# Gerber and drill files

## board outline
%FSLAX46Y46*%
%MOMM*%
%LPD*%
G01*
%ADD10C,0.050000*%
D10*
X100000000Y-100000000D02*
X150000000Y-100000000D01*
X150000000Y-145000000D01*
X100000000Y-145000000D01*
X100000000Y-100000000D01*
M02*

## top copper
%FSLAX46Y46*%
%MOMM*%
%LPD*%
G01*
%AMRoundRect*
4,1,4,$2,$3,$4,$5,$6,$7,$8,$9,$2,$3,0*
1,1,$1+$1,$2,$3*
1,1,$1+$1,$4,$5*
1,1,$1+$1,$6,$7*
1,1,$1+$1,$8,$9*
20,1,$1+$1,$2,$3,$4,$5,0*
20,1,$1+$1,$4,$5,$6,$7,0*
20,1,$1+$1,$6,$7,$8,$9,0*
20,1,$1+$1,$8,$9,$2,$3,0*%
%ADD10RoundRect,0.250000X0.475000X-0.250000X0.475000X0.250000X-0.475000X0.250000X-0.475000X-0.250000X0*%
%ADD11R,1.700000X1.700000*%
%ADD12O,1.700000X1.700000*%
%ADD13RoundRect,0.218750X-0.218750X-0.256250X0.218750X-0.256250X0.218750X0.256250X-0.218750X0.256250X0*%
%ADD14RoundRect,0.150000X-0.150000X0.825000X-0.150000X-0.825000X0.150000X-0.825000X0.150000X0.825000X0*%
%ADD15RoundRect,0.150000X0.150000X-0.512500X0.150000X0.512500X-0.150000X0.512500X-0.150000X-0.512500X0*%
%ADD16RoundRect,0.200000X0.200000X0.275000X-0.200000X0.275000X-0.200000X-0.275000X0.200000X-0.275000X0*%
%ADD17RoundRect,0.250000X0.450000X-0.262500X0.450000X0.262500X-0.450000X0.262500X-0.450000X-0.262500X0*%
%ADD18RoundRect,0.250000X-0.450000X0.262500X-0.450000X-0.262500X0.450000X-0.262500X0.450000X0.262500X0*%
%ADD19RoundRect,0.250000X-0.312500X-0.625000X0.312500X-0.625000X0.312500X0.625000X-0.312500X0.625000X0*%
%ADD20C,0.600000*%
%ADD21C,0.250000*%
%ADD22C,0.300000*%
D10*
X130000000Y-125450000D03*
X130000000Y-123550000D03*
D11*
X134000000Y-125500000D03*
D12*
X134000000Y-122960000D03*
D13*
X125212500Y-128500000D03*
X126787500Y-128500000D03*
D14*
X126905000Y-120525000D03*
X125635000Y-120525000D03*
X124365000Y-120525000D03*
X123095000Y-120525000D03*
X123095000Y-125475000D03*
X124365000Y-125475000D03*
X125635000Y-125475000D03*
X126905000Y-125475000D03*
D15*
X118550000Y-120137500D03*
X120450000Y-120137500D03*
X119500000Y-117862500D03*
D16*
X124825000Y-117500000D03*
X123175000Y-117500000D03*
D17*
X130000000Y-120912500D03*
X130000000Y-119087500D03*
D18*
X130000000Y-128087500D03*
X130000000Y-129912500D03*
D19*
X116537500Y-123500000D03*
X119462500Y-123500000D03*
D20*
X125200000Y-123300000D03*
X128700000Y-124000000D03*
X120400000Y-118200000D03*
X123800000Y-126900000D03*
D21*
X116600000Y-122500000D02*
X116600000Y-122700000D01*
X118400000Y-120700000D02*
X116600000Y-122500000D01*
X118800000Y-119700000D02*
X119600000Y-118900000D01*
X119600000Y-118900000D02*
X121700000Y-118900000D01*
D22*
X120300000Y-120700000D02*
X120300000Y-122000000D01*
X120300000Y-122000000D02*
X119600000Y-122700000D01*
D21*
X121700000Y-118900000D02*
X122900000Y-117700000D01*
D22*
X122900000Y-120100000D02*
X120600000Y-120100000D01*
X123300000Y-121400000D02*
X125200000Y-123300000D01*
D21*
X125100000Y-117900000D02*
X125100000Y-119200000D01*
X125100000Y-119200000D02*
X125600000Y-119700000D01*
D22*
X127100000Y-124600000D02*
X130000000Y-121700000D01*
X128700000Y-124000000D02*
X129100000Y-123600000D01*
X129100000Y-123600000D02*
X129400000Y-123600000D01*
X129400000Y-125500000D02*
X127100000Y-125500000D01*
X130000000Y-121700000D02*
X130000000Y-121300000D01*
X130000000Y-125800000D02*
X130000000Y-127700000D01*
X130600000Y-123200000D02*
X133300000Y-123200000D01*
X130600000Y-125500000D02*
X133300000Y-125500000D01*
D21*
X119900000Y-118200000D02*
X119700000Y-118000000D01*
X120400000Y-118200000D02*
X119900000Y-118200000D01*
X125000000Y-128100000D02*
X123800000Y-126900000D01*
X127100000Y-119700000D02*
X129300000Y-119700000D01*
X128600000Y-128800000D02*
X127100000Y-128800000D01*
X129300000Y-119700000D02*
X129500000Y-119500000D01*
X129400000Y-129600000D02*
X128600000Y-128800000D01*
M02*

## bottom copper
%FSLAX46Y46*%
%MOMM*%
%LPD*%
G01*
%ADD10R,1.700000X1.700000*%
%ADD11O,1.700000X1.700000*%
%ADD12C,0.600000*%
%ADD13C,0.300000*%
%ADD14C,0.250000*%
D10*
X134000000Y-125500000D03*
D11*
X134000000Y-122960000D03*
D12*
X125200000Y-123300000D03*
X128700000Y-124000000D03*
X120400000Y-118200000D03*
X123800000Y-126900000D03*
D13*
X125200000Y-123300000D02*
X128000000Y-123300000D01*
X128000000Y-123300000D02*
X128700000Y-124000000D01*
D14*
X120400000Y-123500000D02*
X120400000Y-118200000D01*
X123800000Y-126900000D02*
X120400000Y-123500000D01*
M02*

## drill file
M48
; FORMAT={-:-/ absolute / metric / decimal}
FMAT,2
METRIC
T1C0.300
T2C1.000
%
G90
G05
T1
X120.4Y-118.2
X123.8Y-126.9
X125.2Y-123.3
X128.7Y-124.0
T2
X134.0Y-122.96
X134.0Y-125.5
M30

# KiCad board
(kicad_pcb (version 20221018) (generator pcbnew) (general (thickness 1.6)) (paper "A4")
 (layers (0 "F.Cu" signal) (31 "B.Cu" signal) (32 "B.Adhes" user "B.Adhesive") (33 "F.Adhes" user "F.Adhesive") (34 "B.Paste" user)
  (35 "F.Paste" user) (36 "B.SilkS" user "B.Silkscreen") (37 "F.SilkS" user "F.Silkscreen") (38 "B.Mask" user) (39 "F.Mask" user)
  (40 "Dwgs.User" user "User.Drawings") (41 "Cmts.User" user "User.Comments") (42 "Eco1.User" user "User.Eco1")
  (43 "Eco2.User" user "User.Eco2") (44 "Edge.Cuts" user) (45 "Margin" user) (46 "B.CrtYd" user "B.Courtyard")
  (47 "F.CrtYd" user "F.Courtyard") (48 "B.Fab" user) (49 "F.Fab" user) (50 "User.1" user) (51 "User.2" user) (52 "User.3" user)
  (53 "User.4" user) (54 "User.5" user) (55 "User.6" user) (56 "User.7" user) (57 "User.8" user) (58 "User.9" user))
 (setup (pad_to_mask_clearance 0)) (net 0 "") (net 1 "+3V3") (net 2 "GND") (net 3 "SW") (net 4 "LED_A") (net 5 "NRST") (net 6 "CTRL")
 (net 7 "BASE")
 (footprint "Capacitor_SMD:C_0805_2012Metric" (layer "F.Cu") (at 130 124.5 90)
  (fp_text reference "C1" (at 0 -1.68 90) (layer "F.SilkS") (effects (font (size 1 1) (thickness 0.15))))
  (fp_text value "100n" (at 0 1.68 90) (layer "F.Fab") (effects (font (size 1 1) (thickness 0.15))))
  (pad "1" smd roundrect (at -0.95 0 90) (size 1 1.45) (layers "F.Cu" "F.Paste" "F.Mask") (roundrect_rratio 0.25) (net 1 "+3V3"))
  (pad "2" smd roundrect (at 0.95 0 90) (size 1 1.45) (layers "F.Cu" "F.Paste" "F.Mask") (roundrect_rratio 0.25) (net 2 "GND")))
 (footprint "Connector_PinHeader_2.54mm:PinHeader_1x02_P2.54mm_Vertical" (layer "F.Cu") (at 134 125.5 180)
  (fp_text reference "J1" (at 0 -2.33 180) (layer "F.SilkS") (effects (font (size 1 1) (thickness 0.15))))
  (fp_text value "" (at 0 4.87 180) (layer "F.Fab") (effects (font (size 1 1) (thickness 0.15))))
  (pad "1" thru_hole rect (at 0 0 180) (size 1.7 1.7) (drill 1) (layers "*.Cu" "*.Mask") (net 1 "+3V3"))
  (pad "2" thru_hole oval (at 0 2.54 180) (size 1.7 1.7) (drill 1) (layers "*.Cu" "*.Mask") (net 2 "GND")))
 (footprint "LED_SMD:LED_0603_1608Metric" (layer "F.Cu") (at 126 128.5)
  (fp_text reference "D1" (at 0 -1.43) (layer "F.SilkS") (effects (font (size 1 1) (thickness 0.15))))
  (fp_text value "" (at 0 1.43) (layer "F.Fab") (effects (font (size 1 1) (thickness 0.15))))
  (pad "1" smd roundrect (at -0.7875 0) (size 0.875 0.95) (layers "F.Cu" "F.Paste" "F.Mask") (roundrect_rratio 0.25) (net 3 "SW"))
  (pad "2" smd roundrect (at 0.7875 0) (size 0.875 0.95) (layers "F.Cu" "F.Paste" "F.Mask") (roundrect_rratio 0.25) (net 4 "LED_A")))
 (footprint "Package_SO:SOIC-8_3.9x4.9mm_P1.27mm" (layer "F.Cu") (at 125 123 -90)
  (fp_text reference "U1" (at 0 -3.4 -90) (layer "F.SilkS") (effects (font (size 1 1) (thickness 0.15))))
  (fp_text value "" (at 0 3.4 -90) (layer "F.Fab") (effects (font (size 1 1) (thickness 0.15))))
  (pad "1" smd roundrect (at -2.475 -1.905 270) (size 1.95 0.6) (layers "F.Cu" "F.Paste" "F.Mask") (roundrect_rratio 0.25) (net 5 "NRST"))
  (pad "2" smd roundrect (at -2.475 -0.635 270) (size 1.95 0.6) (layers "F.Cu" "F.Paste" "F.Mask") (roundrect_rratio 0.25) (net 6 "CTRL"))
  (pad "3" smd roundrect (at -2.475 0.635 270) (size 1.95 0.6) (layers "F.Cu" "F.Paste" "F.Mask") (roundrect_rratio 0.25))
  (pad "4" smd roundrect (at -2.475 1.905 270) (size 1.95 0.6) (layers "F.Cu" "F.Paste" "F.Mask") (roundrect_rratio 0.25) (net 2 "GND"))
  (pad "5" smd roundrect (at 2.475 1.905 270) (size 1.95 0.6) (layers "F.Cu" "F.Paste" "F.Mask") (roundrect_rratio 0.25))
  (pad "6" smd roundrect (at 2.475 0.635 270) (size 1.95 0.6) (layers "F.Cu" "F.Paste" "F.Mask") (roundrect_rratio 0.25))
  (pad "7" smd roundrect (at 2.475 -0.635 270) (size 1.95 0.6) (layers "F.Cu" "F.Paste" "F.Mask") (roundrect_rratio 0.25))
  (pad "8" smd roundrect (at 2.475 -1.905 270) (size 1.95 0.6) (layers "F.Cu" "F.Paste" "F.Mask") (roundrect_rratio 0.25) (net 1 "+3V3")))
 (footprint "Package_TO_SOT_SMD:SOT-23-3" (layer "F.Cu") (at 119.5 119 90)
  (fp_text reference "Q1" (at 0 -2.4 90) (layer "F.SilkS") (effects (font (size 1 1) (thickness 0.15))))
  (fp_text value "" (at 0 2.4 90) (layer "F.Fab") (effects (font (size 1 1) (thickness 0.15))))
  (pad "1" smd roundrect (at -1.1375 -0.95 90) (size 1.325 0.6) (layers "F.Cu" "F.Paste" "F.Mask") (roundrect_rratio 0.25) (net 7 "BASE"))
  (pad "2" smd roundrect (at -1.1375 0.95 90) (size 1.325 0.6) (layers "F.Cu" "F.Paste" "F.Mask") (roundrect_rratio 0.25) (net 2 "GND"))
  (pad "3" smd roundrect (at 1.1375 0 90) (size 1.325 0.6) (layers "F.Cu" "F.Paste" "F.Mask") (roundrect_rratio 0.25) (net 3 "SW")))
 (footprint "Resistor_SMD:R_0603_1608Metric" (layer "F.Cu") (at 124 117.5 180)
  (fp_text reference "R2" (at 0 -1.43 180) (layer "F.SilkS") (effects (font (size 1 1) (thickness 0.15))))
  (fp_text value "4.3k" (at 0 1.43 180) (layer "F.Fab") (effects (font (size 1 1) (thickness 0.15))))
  (pad "1" smd roundrect (at -0.825 0 180) (size 0.8 0.95) (layers "F.Cu" "F.Paste" "F.Mask") (roundrect_rratio 0.25) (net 6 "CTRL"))
  (pad "2" smd roundrect (at 0.825 0 180) (size 0.8 0.95) (layers "F.Cu" "F.Paste" "F.Mask") (roundrect_rratio 0.25) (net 7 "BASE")))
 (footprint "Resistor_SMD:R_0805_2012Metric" (layer "F.Cu") (at 130 120 90)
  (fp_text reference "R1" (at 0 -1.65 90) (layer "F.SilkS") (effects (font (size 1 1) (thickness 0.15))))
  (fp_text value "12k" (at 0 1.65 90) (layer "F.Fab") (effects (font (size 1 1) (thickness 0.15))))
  (pad "1" smd roundrect (at -0.9125 0 90) (size 1.025 1.4) (layers "F.Cu" "F.Paste" "F.Mask") (roundrect_rratio 0.243902) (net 1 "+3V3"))
  (pad "2" smd roundrect (at 0.9125 0 90) (size 1.025 1.4) (layers "F.Cu" "F.Paste" "F.Mask") (roundrect_rratio 0.243902) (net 5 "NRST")))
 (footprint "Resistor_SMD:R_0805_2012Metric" (layer "F.Cu") (at 130 129 -90)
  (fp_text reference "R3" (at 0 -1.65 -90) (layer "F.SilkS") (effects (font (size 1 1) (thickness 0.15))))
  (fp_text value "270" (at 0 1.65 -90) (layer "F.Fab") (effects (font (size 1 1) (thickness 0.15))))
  (pad "1" smd roundrect (at -0.9125 0 270) (size 1.025 1.4) (layers "F.Cu" "F.Paste" "F.Mask") (roundrect_rratio 0.243902) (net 1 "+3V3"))
  (pad "2" smd roundrect (at 0.9125 0 270) (size 1.025 1.4) (layers "F.Cu" "F.Paste" "F.Mask") (roundrect_rratio 0.243902) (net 4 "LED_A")))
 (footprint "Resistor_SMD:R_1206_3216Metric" (layer "F.Cu") (at 118 123.5)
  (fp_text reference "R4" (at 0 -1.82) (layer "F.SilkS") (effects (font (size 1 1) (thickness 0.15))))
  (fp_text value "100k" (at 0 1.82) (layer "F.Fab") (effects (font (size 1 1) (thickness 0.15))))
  (pad "1" smd roundrect (at -1.4625 0) (size 1.125 1.75) (layers "F.Cu" "F.Paste" "F.Mask") (roundrect_rratio 0.222222) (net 7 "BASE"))
  (pad "2" smd roundrect (at 1.4625 0) (size 1.125 1.75) (layers "F.Cu" "F.Paste" "F.Mask") (roundrect_rratio 0.222222) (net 2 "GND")))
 (gr_rect (start 100 100) (end 150 145) (stroke (width 0.05) (type default)) (fill none) (layer "Edge.Cuts"))
 (segment (start 116.6 122.5) (end 116.6 122.7) (width 0.25) (layer "F.Cu") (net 7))
 (segment (start 118.4 120.7) (end 116.6 122.5) (width 0.25) (layer "F.Cu") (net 7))
 (segment (start 118.8 119.7) (end 119.6 118.9) (width 0.25) (layer "F.Cu") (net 7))
 (segment (start 119.6 118.9) (end 121.7 118.9) (width 0.25) (layer "F.Cu") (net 7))
 (segment (start 120.3 120.7) (end 120.3 122) (width 0.3) (layer "F.Cu") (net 2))
 (segment (start 120.3 122) (end 119.6 122.7) (width 0.3) (layer "F.Cu") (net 2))
 (segment (start 121.7 118.9) (end 122.9 117.7) (width 0.25) (layer "F.Cu") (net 7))
 (segment (start 122.9 120.1) (end 120.6 120.1) (width 0.3) (layer "F.Cu") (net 2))
 (segment (start 123.3 121.4) (end 125.2 123.3) (width 0.3) (layer "F.Cu") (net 2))
 (segment (start 125.1 117.9) (end 125.1 119.2) (width 0.25) (layer "F.Cu") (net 6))
 (segment (start 125.1 119.2) (end 125.6 119.7) (width 0.25) (layer "F.Cu") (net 6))
 (segment (start 127.1 124.6) (end 130 121.7) (width 0.3) (layer "F.Cu") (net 1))
 (segment (start 128.7 124) (end 129.1 123.6) (width 0.3) (layer "F.Cu") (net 2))
 (segment (start 129.1 123.6) (end 129.4 123.6) (width 0.3) (layer "F.Cu") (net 2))
 (segment (start 129.4 125.5) (end 127.1 125.5) (width 0.3) (layer "F.Cu") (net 1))
 (segment (start 130 121.7) (end 130 121.3) (width 0.3) (layer "F.Cu") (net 1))
 (segment (start 130 125.8) (end 130 127.7) (width 0.3) (layer "F.Cu") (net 1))
 (segment (start 130.6 123.2) (end 133.3 123.2) (width 0.3) (layer "F.Cu") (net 2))
 (segment (start 130.6 125.5) (end 133.3 125.5) (width 0.3) (layer "F.Cu") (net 1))
 (via (at 125.2 123.3) (size 0.6) (drill 0.3) (layers "F.Cu" "B.Cu") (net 2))
 (via (at 128.7 124) (size 0.6) (drill 0.3) (layers "F.Cu" "B.Cu") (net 2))
 (segment (start 119.9 118.2) (end 119.7 118) (width 0.25) (layer "F.Cu") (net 3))
 (segment (start 120.4 118.2) (end 119.9 118.2) (width 0.25) (layer "F.Cu") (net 3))
 (segment (start 125 128.1) (end 123.8 126.9) (width 0.25) (layer "F.Cu") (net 3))
 (segment (start 125.2 123.3) (end 128 123.3) (width 0.3) (layer "B.Cu") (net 2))
 (segment (start 127.1 119.7) (end 129.3 119.7) (width 0.25) (layer "F.Cu") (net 5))
 (segment (start 128 123.3) (end 128.7 124) (width 0.3) (layer "B.Cu") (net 2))
 (segment (start 128.6 128.8) (end 127.1 128.8) (width 0.25) (layer "F.Cu") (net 4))
 (segment (start 129.3 119.7) (end 129.5 119.5) (width 0.25) (layer "F.Cu") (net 5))
 (segment (start 129.4 129.6) (end 128.6 128.8) (width 0.25) (layer "F.Cu") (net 4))
 (via (at 120.4 118.2) (size 0.6) (drill 0.3) (layers "F.Cu" "B.Cu") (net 3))
 (via (at 123.8 126.9) (size 0.6) (drill 0.3) (layers "F.Cu" "B.Cu") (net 3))
 (segment (start 120.4 123.5) (end 120.4 118.2) (width 0.25) (layer "B.Cu") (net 3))
 (segment (start 123.8 126.9) (end 120.4 123.5) (width 0.25) (layer "B.Cu") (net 3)))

